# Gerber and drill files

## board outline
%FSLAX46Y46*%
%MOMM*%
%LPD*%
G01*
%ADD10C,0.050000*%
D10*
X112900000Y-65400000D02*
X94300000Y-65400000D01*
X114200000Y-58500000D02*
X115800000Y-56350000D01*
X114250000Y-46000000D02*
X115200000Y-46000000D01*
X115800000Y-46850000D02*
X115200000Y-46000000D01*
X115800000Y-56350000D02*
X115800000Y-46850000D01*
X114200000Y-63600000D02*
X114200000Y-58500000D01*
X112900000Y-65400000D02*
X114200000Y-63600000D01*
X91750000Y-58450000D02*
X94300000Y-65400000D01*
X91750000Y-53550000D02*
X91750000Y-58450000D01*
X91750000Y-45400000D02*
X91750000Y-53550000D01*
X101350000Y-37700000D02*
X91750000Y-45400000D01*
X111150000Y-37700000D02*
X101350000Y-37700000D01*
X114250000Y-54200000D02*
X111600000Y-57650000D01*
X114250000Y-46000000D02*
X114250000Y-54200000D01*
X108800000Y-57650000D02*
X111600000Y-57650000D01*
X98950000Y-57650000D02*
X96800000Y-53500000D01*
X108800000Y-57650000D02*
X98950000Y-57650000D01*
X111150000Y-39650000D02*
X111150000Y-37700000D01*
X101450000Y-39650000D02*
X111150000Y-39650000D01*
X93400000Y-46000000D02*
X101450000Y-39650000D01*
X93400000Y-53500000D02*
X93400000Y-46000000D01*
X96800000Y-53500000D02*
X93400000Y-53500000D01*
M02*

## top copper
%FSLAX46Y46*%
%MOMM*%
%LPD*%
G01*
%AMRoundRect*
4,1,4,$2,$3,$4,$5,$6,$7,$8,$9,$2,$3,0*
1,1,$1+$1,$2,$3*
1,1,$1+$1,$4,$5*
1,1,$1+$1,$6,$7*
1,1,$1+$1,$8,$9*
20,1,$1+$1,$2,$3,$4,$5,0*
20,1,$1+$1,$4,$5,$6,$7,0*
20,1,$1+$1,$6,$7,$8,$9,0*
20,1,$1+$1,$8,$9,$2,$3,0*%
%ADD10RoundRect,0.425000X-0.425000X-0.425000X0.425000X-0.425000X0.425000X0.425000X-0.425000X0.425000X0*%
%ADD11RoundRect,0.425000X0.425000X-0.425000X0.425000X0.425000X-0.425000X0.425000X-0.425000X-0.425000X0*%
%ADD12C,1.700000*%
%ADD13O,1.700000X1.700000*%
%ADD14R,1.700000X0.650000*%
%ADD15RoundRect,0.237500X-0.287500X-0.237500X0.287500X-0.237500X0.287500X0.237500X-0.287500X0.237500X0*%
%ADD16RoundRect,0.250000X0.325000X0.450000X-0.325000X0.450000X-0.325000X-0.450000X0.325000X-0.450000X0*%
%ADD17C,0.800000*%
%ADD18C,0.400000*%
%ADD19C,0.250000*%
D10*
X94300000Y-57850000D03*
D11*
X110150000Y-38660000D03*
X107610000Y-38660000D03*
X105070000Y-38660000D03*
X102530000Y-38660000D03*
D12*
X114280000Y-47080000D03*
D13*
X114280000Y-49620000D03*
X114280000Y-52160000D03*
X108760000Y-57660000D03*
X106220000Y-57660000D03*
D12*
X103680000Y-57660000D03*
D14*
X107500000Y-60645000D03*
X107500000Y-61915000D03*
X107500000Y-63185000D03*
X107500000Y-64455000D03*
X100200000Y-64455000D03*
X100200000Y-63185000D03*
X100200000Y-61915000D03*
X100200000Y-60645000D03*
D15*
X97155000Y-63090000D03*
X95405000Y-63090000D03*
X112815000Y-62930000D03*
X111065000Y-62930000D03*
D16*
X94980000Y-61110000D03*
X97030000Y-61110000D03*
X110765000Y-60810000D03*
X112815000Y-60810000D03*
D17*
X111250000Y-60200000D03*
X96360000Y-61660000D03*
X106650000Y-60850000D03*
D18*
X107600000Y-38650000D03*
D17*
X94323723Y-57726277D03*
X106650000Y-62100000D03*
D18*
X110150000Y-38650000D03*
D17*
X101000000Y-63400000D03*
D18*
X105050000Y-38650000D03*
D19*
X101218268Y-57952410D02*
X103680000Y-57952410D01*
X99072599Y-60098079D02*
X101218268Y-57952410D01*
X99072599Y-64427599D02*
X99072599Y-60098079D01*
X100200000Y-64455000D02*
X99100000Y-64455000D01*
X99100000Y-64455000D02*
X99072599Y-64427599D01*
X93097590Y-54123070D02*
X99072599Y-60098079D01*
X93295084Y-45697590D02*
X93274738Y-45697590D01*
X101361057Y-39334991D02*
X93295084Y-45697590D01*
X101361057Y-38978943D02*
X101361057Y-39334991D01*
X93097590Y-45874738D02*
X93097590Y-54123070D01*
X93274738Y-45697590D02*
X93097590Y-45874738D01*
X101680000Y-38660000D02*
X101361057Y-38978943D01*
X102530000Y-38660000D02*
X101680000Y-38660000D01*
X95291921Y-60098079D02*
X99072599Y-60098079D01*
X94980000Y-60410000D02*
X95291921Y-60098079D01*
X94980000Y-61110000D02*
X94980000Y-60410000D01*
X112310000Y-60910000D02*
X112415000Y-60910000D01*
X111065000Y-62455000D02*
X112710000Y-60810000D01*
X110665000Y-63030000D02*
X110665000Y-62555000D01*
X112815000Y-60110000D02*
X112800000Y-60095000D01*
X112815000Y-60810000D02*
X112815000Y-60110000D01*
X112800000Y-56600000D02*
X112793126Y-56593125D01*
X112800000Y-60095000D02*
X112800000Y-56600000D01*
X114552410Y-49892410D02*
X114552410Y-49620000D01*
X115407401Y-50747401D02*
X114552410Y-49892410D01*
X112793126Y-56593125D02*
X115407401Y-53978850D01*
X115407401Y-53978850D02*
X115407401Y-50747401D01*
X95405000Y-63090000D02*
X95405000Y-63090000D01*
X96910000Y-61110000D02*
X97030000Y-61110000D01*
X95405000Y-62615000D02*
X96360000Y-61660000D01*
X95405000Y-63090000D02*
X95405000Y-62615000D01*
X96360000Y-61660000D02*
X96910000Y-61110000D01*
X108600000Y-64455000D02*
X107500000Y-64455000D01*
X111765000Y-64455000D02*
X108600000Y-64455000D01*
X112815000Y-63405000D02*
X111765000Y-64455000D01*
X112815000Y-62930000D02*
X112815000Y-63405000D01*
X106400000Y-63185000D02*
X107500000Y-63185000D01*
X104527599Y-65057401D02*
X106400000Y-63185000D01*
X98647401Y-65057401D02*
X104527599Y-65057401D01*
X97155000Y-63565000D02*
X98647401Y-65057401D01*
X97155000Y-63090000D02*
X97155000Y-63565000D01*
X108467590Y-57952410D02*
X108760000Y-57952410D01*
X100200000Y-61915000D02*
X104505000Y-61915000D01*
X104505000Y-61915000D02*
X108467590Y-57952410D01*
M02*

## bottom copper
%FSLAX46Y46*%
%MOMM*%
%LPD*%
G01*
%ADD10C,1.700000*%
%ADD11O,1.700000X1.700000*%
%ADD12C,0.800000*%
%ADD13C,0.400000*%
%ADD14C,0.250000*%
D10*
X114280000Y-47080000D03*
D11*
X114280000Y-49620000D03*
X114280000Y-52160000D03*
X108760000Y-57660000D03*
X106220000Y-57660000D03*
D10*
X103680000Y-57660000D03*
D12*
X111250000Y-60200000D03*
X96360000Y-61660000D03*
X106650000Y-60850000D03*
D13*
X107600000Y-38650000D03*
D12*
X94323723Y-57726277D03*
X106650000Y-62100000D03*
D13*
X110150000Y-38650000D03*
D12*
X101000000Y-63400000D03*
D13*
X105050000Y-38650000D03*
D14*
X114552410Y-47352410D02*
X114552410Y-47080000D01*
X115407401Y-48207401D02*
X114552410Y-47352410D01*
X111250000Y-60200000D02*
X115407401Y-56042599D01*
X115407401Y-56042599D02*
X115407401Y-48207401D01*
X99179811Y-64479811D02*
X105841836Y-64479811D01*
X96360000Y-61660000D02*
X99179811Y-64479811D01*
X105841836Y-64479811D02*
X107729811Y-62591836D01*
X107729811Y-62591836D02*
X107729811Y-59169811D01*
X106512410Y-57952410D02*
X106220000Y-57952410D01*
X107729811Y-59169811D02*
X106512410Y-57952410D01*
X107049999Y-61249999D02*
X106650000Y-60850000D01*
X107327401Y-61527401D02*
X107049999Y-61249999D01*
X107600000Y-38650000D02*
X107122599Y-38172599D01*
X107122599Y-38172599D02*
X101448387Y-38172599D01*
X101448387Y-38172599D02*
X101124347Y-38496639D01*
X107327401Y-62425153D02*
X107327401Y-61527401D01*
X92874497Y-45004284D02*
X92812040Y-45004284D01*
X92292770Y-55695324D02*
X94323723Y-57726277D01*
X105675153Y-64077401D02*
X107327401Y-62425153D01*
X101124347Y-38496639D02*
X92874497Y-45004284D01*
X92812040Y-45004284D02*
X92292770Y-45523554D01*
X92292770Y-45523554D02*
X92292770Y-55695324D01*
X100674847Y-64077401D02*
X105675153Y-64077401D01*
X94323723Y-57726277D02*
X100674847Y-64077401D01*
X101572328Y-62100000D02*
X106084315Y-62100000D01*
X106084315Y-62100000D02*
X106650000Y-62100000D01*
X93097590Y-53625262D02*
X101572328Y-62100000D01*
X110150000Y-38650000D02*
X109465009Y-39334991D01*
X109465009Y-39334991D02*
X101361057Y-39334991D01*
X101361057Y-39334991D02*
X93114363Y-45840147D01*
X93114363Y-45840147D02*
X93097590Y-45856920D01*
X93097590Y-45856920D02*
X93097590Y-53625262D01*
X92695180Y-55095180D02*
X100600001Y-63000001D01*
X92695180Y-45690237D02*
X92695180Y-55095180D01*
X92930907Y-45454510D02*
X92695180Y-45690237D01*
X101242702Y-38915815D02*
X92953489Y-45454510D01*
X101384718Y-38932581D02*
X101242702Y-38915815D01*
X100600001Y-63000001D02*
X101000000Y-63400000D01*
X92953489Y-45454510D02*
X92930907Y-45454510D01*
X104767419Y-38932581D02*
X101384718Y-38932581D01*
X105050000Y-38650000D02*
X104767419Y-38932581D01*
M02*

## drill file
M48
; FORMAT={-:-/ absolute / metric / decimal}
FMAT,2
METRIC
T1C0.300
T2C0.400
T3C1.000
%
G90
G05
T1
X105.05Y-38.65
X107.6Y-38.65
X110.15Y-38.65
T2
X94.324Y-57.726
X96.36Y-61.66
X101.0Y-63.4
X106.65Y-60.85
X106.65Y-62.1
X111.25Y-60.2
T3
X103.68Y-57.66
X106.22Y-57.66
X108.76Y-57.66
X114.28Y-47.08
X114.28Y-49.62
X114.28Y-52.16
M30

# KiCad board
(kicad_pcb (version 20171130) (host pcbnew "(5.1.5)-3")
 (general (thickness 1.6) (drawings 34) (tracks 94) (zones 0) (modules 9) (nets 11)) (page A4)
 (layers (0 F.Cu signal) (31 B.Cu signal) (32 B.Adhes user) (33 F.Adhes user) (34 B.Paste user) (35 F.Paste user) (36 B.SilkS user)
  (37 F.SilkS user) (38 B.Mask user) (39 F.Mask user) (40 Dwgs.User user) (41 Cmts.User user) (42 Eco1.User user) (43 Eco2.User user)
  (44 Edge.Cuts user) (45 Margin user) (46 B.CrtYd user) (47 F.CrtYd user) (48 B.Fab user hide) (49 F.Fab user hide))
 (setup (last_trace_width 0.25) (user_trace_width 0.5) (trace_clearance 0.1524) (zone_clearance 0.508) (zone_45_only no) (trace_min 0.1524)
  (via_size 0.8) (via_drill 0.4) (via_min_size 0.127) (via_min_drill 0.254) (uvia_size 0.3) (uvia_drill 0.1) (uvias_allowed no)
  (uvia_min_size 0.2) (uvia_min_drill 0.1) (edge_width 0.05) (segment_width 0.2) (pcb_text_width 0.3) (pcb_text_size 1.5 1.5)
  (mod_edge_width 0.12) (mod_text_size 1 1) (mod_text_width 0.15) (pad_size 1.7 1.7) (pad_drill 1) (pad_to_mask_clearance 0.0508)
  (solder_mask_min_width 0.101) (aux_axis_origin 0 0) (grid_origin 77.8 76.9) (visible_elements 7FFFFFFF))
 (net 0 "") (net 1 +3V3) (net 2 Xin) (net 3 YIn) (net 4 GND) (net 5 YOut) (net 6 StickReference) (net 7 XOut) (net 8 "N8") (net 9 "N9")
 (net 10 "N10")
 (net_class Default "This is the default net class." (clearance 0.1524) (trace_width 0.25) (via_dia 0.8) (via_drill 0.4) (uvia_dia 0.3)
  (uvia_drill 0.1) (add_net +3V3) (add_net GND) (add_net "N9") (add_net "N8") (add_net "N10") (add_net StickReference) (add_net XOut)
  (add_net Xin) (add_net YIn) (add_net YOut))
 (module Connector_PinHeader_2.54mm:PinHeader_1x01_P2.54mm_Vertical (layer F.Cu) (at 94.3 57.85)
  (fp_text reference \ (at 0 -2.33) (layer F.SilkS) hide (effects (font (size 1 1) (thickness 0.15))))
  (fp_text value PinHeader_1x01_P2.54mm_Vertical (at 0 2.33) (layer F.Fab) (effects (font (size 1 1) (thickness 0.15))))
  (pad 1 smd roundrect (at 0 0) (size 1.7 1.7) (layers F.Cu F.Paste F.Mask) (roundrect_rratio 0.25) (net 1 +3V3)))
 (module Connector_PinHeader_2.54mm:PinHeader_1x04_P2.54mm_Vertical (layer F.Cu) (at 102.53 38.66 90)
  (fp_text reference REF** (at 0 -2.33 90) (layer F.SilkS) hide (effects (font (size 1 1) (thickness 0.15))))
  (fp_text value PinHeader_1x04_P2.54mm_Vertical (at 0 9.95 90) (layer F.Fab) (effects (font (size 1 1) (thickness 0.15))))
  (pad 4 smd roundrect (at 0 7.62 90) (size 1.7 1.7) (layers F.Cu F.Paste F.Mask) (roundrect_rratio 0.25) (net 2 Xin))
  (pad 3 smd roundrect (at 0 5.08 90) (size 1.7 1.7) (layers F.Cu F.Paste F.Mask) (roundrect_rratio 0.25) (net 1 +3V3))
  (pad 2 smd roundrect (at 0 2.54 90) (size 1.7 1.7) (layers F.Cu F.Paste F.Mask) (roundrect_rratio 0.25) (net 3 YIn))
  (pad 1 smd roundrect (at 0 0 90) (size 1.7 1.7) (layers F.Cu F.Paste F.Mask) (roundrect_rratio 0.25) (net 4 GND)))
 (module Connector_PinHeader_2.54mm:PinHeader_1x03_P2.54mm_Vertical (layer F.Cu) (at 114.28 47.08)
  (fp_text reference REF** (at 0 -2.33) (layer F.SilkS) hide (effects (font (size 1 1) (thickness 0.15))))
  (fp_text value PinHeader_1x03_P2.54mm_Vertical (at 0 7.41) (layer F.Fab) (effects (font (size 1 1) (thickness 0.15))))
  (pad 1 thru_hole circle (at 0 0) (size 1.7 1.7) (drill 1) (layers *.Cu *.Mask) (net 4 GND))
  (pad 2 thru_hole oval (at 0 2.54) (size 1.7 1.7) (drill 1) (layers *.Cu *.Mask) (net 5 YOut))
  (pad 3 thru_hole oval (at 0 5.08) (size 1.7 1.7) (drill 1) (layers *.Cu *.Mask)))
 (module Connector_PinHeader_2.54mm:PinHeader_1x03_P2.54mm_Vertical (layer F.Cu) (at 103.68 57.66 90)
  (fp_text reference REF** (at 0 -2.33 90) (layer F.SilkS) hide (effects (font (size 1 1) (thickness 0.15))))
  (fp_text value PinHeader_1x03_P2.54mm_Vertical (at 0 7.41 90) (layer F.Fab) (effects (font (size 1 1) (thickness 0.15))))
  (pad 3 thru_hole oval (at 0 5.08 90) (size 1.7 1.7) (drill 1) (layers *.Cu *.Mask) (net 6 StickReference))
  (pad 2 thru_hole oval (at 0 2.54 90) (size 1.7 1.7) (drill 1) (layers *.Cu *.Mask) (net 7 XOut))
  (pad 1 thru_hole circle (at 0 0 90) (size 1.7 1.7) (drill 1) (layers *.Cu *.Mask) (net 4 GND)))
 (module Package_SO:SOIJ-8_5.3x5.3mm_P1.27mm (layer F.Cu) (at 103.85 62.55)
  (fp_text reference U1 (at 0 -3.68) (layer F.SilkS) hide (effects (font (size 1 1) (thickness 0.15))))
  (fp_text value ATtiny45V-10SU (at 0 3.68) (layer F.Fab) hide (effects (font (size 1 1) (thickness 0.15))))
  (pad 8 smd rect (at 3.65 -1.905) (size 1.7 0.65) (layers F.Cu F.Paste F.Mask) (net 1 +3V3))
  (pad 7 smd rect (at 3.65 -0.635) (size 1.7 0.65) (layers F.Cu F.Paste F.Mask) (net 2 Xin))
  (pad 6 smd rect (at 3.65 0.635) (size 1.7 0.65) (layers F.Cu F.Paste F.Mask) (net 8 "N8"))
  (pad 5 smd rect (at 3.65 1.905) (size 1.7 0.65) (layers F.Cu F.Paste F.Mask) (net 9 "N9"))
  (pad 4 smd rect (at -3.65 1.905) (size 1.7 0.65) (layers F.Cu F.Paste F.Mask) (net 4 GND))
  (pad 3 smd rect (at -3.65 0.635) (size 1.7 0.65) (layers F.Cu F.Paste F.Mask) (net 3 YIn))
  (pad 2 smd rect (at -3.65 -0.635) (size 1.7 0.65) (layers F.Cu F.Paste F.Mask) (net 6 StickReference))
  (pad 1 smd rect (at -3.65 -1.905) (size 1.7 0.65) (layers F.Cu F.Paste F.Mask) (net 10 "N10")))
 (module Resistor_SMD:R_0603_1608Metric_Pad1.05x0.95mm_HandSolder (layer F.Cu) (at 96.28 63.09)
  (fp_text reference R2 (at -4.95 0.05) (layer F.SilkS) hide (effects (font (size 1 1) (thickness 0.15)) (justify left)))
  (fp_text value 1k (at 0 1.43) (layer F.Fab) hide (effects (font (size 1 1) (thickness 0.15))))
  (pad 2 smd roundrect (at 0.875 0) (size 1.05 0.95) (layers F.Cu F.Paste F.Mask) (roundrect_rratio 0.25) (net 8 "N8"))
  (pad 1 smd roundrect (at -0.875 0) (size 1.05 0.95) (layers F.Cu F.Paste F.Mask) (roundrect_rratio 0.25) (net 7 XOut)))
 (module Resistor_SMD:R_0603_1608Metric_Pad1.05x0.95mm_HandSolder (layer F.Cu) (at 111.94 62.93)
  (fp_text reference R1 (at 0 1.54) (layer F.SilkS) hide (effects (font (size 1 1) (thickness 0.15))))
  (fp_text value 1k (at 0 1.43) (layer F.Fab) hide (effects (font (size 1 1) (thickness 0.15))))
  (pad 2 smd roundrect (at 0.875 0) (size 1.05 0.95) (layers F.Cu F.Paste F.Mask) (roundrect_rratio 0.25) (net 9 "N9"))
  (pad 1 smd roundrect (at -0.875 0) (size 1.05 0.95) (layers F.Cu F.Paste F.Mask) (roundrect_rratio 0.25) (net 5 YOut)))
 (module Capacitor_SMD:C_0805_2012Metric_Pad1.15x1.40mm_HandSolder (layer F.Cu) (at 96.005 61.11 180)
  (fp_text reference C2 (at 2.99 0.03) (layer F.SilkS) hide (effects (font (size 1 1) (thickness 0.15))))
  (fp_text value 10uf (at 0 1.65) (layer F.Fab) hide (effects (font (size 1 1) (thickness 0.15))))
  (pad 2 smd roundrect (at 1.025 0 180) (size 1.15 1.4) (layers F.Cu F.Paste F.Mask) (roundrect_rratio 0.217391) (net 4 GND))
  (pad 1 smd roundrect (at -1.025 0 180) (size 1.15 1.4) (layers F.Cu F.Paste F.Mask) (roundrect_rratio 0.217391) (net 7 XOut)))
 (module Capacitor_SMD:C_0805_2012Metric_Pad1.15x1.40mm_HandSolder (layer F.Cu) (at 111.79 60.81 180)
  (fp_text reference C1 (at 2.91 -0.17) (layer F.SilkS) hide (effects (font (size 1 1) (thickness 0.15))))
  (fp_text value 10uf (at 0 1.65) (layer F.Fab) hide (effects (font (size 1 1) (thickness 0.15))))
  (pad 2 smd roundrect (at 1.025 0 180) (size 1.15 1.4) (layers F.Cu F.Paste F.Mask) (roundrect_rratio 0.217391) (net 4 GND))
  (pad 1 smd roundrect (at -1.025 0 180) (size 1.15 1.4) (layers F.Cu F.Paste F.Mask) (roundrect_rratio 0.217391) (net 5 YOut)))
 (gr_line (start 112.9 65.4) (end 94.3 65.4) (layer Edge.Cuts) (width 0.05))
 (gr_line (start 114.2 58.5) (end 115.8 56.35) (layer Edge.Cuts) (width 0.05))
 (gr_line (start 114.25 46) (end 115.2 46) (layer Edge.Cuts) (width 0.05))
 (gr_line (start 115.8 46.85) (end 115.2 46) (layer Edge.Cuts) (width 0.05))
 (gr_line (start 115.8 56.35) (end 115.8 46.85) (layer Edge.Cuts) (width 0.05))
 (gr_line (start 114.2 63.6) (end 114.2 58.5) (layer Edge.Cuts) (width 0.05))
 (gr_line (start 112.9 65.4) (end 114.2 63.6) (layer Edge.Cuts) (width 0.05))
 (gr_line (start 91.75 58.45) (end 94.3 65.4) (layer Edge.Cuts) (width 0.05))
 (gr_line (start 91.75 53.55) (end 91.75 58.45) (layer Edge.Cuts) (width 0.05))
 (gr_line (start 91.75 45.4) (end 91.75 53.55) (layer Edge.Cuts) (width 0.05))
 (gr_line (start 101.35 37.7) (end 91.75 45.4) (layer Edge.Cuts) (width 0.05))
 (gr_line (start 111.15 37.7) (end 101.35 37.7) (layer Edge.Cuts) (width 0.05))
 (gr_line (start 114.25 54.2) (end 111.6 57.65) (layer Edge.Cuts) (width 0.05))
 (gr_line (start 114.25 46) (end 114.25 54.2) (layer Edge.Cuts) (width 0.05))
 (gr_line (start 108.8 57.65) (end 111.6 57.65) (layer Edge.Cuts) (width 0.05))
 (gr_line (start 98.95 57.65) (end 96.8 53.5) (layer Edge.Cuts) (width 0.05))
 (gr_line (start 108.8 57.65) (end 98.95 57.65) (layer Edge.Cuts) (width 0.05))
 (gr_line (start 111.15 39.65) (end 111.15 37.7) (layer Edge.Cuts) (width 0.05))
 (gr_line (start 101.45 39.65) (end 111.15 39.65) (layer Edge.Cuts) (width 0.05))
 (gr_line (start 93.4 46) (end 101.45 39.65) (layer Edge.Cuts) (width 0.05))
 (gr_line (start 93.4 53.5) (end 93.4 46) (layer Edge.Cuts) (width 0.05))
 (gr_line (start 96.8 53.5) (end 93.4 53.5) (layer Edge.Cuts) (width 0.05))
 (via (at 111.25 60.2) (size 0.8) (drill 0.4) (layers F.Cu B.Cu) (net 4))
 (segment (start 101.218268 57.95241) (end 103.68 57.95241) (width 0.25) (layer F.Cu) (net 4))
 (segment (start 99.072599 60.098079) (end 101.218268 57.95241) (width 0.25) (layer F.Cu) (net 4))
 (segment (start 99.072599 64.427599) (end 99.072599 60.098079) (width 0.25) (layer F.Cu) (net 4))
 (segment (start 100.2 64.455) (end 99.1 64.455) (width 0.25) (layer F.Cu) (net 4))
 (segment (start 99.1 64.455) (end 99.072599 64.427599) (width 0.25) (layer F.Cu) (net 4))
 (segment (start 93.09759 54.12307) (end 99.072599 60.098079) (width 0.25) (layer F.Cu) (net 4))
 (segment (start 93.295084 45.69759) (end 93.274738 45.69759) (width 0.25) (layer F.Cu) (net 4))
 (segment (start 101.361057 39.334991) (end 93.295084 45.69759) (width 0.25) (layer F.Cu) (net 4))
 (segment (start 101.361057 38.978943) (end 101.361057 39.334991) (width 0.25) (layer F.Cu) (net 4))
 (segment (start 93.09759 45.874738) (end 93.09759 54.12307) (width 0.25) (layer F.Cu) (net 4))
 (segment (start 93.274738 45.69759) (end 93.09759 45.874738) (width 0.25) (layer F.Cu) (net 4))
 (segment (start 101.68 38.66) (end 101.361057 38.978943) (width 0.25) (layer F.Cu) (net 4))
 (segment (start 102.53 38.66) (end 101.68 38.66) (width 0.25) (layer F.Cu) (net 4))
 (segment (start 95.291921 60.098079) (end 99.072599 60.098079) (width 0.25) (layer F.Cu) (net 4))
 (segment (start 94.98 60.41) (end 95.291921 60.098079) (width 0.25) (layer F.Cu) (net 4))
 (segment (start 94.98 61.11) (end 94.98 60.41) (width 0.25) (layer F.Cu) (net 4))
 (segment (start 114.55241 47.35241) (end 114.55241 47.08) (width 0.25) (layer B.Cu) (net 4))
 (segment (start 115.407401 48.207401) (end 114.55241 47.35241) (width 0.25) (layer B.Cu) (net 4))
 (segment (start 111.25 60.2) (end 115.407401 56.042599) (width 0.25) (layer B.Cu) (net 4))
 (segment (start 115.407401 56.042599) (end 115.407401 48.207401) (width 0.25) (layer B.Cu) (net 4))
 (segment (start 112.31 60.91) (end 112.415 60.91) (width 0.25) (layer F.Cu) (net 5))
 (segment (start 111.065 62.455) (end 112.71 60.81) (width 0.25) (layer F.Cu) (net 5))
 (segment (start 110.665 63.03) (end 110.665 62.555) (width 0.25) (layer F.Cu) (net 5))
 (segment (start 112.815 60.11) (end 112.8 60.095) (width 0.25) (layer F.Cu) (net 5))
 (segment (start 112.815 60.81) (end 112.815 60.11) (width 0.25) (layer F.Cu) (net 5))
 (segment (start 112.8 56.6) (end 112.793126 56.593125) (width 0.25) (layer F.Cu) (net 5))
 (segment (start 112.8 60.095) (end 112.8 56.6) (width 0.25) (layer F.Cu) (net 5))
 (segment (start 114.55241 49.89241) (end 114.55241 49.62) (width 0.25) (layer F.Cu) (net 5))
 (segment (start 115.407401 50.747401) (end 114.55241 49.89241) (width 0.25) (layer F.Cu) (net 5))
 (segment (start 112.793126 56.593125) (end 115.407401 53.97885) (width 0.25) (layer F.Cu) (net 5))
 (segment (start 115.407401 53.97885) (end 115.407401 50.747401) (width 0.25) (layer F.Cu) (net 5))
 (segment (start 95.405 63.09) (end 95.405 63.09) (width 0.25) (layer F.Cu) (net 7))
 (segment (start 96.91 61.11) (end 97.03 61.11) (width 0.25) (layer F.Cu) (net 7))
 (segment (start 95.405 62.615) (end 96.36 61.66) (width 0.25) (layer F.Cu) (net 7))
 (segment (start 95.405 63.09) (end 95.405 62.615) (width 0.25) (layer F.Cu) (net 7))
 (segment (start 96.36 61.66) (end 96.91 61.11) (width 0.25) (layer F.Cu) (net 7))
 (via (at 96.36 61.66) (size 0.8) (drill 0.4) (layers F.Cu B.Cu) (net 7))
 (segment (start 99.179811 64.479811) (end 105.841836 64.479811) (width 0.25) (layer B.Cu) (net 7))
 (segment (start 96.36 61.66) (end 99.179811 64.479811) (width 0.25) (layer B.Cu) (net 7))
 (segment (start 105.841836 64.479811) (end 107.729811 62.591836) (width 0.25) (layer B.Cu) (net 7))
 (segment (start 107.729811 62.591836) (end 107.729811 59.169811) (width 0.25) (layer B.Cu) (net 7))
 (segment (start 106.51241 57.95241) (end 106.22 57.95241) (width 0.25) (layer B.Cu) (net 7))
 (segment (start 107.729811 59.169811) (end 106.51241 57.95241) (width 0.25) (layer B.Cu) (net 7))
 (segment (start 108.6 64.455) (end 107.5 64.455) (width 0.25) (layer F.Cu) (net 9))
 (segment (start 111.765 64.455) (end 108.6 64.455) (width 0.25) (layer F.Cu) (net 9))
 (segment (start 112.815 63.405) (end 111.765 64.455) (width 0.25) (layer F.Cu) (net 9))
 (segment (start 112.815 62.93) (end 112.815 63.405) (width 0.25) (layer F.Cu) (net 9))
 (segment (start 106.4 63.185) (end 107.5 63.185) (width 0.25) (layer F.Cu) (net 8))
 (segment (start 104.527599 65.057401) (end 106.4 63.185) (width 0.25) (layer F.Cu) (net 8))
 (segment (start 98.647401 65.057401) (end 104.527599 65.057401) (width 0.25) (layer F.Cu) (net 8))
 (segment (start 97.155 63.565) (end 98.647401 65.057401) (width 0.25) (layer F.Cu) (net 8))
 (segment (start 97.155 63.09) (end 97.155 63.565) (width 0.25) (layer F.Cu) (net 8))
 (via (at 106.65 60.85) (size 0.8) (drill 0.4) (layers F.Cu B.Cu) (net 1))
 (via (at 107.6 38.65) (size 0.4) (drill 0.3) (layers F.Cu B.Cu) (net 1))
 (segment (start 107.049999 61.249999) (end 106.65 60.85) (width 0.25) (layer B.Cu) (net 1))
 (segment (start 107.327401 61.527401) (end 107.049999 61.249999) (width 0.25) (layer B.Cu) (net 1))
 (segment (start 107.6 38.65) (end 107.122599 38.172599) (width 0.25) (layer B.Cu) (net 1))
 (segment (start 107.122599 38.172599) (end 101.448387 38.172599) (width 0.25) (layer B.Cu) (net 1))
 (segment (start 101.448387 38.172599) (end 101.124347 38.496639) (width 0.25) (layer B.Cu) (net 1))
 (segment (start 107.327401 62.425153) (end 107.327401 61.527401) (width 0.25) (layer B.Cu) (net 1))
 (segment (start 92.874497 45.004284) (end 92.81204 45.004284) (width 0.25) (layer B.Cu) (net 1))
 (segment (start 92.29277 55.695324) (end 94.323723 57.726277) (width 0.25) (layer B.Cu) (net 1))
 (segment (start 105.675153 64.077401) (end 107.327401 62.425153) (width 0.25) (layer B.Cu) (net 1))
 (segment (start 101.124347 38.496639) (end 92.874497 45.004284) (width 0.25) (layer B.Cu) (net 1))
 (segment (start 92.81204 45.004284) (end 92.29277 45.523554) (width 0.25) (layer B.Cu) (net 1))
 (segment (start 92.29277 45.523554) (end 92.29277 55.695324) (width 0.25) (layer B.Cu) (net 1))
 (segment (start 100.674847 64.077401) (end 105.675153 64.077401) (width 0.25) (layer B.Cu) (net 1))
 (segment (start 94.323723 57.726277) (end 100.674847 64.077401) (width 0.25) (layer B.Cu) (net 1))
 (via (at 94.323723 57.726277) (size 0.8) (drill 0.4) (layers F.Cu B.Cu) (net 1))
 (via (at 106.65 62.1) (size 0.8) (drill 0.4) (layers F.Cu B.Cu) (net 2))
 (via (at 110.15 38.65) (size 0.4) (drill 0.3) (layers F.Cu B.Cu) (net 2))
 (segment (start 101.572328 62.1) (end 106.084315 62.1) (width 0.25) (layer B.Cu) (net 2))
 (segment (start 106.084315 62.1) (end 106.65 62.1) (width 0.25) (layer B.Cu) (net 2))
 (segment (start 93.09759 53.625262) (end 101.572328 62.1) (width 0.25) (layer B.Cu) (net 2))
 (segment (start 110.15 38.65) (end 109.465009 39.334991) (width 0.25) (layer B.Cu) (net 2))
 (segment (start 109.465009 39.334991) (end 101.361057 39.334991) (width 0.25) (layer B.Cu) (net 2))
 (segment (start 101.361057 39.334991) (end 93.114363 45.840147) (width 0.25) (layer B.Cu) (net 2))
 (segment (start 93.114363 45.840147) (end 93.09759 45.85692) (width 0.25) (layer B.Cu) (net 2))
 (segment (start 93.09759 45.85692) (end 93.09759 53.625262) (width 0.25) (layer B.Cu) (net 2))
 (via (at 101 63.4) (size 0.8) (drill 0.4) (layers F.Cu B.Cu) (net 3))
 (via (at 105.05 38.65) (size 0.4) (drill 0.3) (layers F.Cu B.Cu) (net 3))
 (segment (start 92.69518 55.09518) (end 100.600001 63.000001) (width 0.25) (layer B.Cu) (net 3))
 (segment (start 92.69518 45.690237) (end 92.69518 55.09518) (width 0.25) (layer B.Cu) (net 3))
 (segment (start 92.930907 45.45451) (end 92.69518 45.690237) (width 0.25) (layer B.Cu) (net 3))
 (segment (start 101.242702 38.915815) (end 92.953489 45.45451) (width 0.25) (layer B.Cu) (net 3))
 (segment (start 101.384718 38.932581) (end 101.242702 38.915815) (width 0.25) (layer B.Cu) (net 3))
 (segment (start 100.600001 63.000001) (end 101 63.4) (width 0.25) (layer B.Cu) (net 3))
 (segment (start 92.953489 45.45451) (end 92.930907 45.45451) (width 0.25) (layer B.Cu) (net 3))
 (segment (start 104.767419 38.932581) (end 101.384718 38.932581) (width 0.25) (layer B.Cu) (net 3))
 (segment (start 105.05 38.65) (end 104.767419 38.932581) (width 0.25) (layer B.Cu) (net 3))
 (segment (start 108.46759 57.95241) (end 108.76 57.95241) (width 0.25) (layer F.Cu) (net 6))
 (segment (start 100.2 61.915) (end 104.505 61.915) (width 0.25) (layer F.Cu) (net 6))
 (segment (start 104.505 61.915) (end 108.46759 57.95241) (width 0.25) (layer F.Cu) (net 6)))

